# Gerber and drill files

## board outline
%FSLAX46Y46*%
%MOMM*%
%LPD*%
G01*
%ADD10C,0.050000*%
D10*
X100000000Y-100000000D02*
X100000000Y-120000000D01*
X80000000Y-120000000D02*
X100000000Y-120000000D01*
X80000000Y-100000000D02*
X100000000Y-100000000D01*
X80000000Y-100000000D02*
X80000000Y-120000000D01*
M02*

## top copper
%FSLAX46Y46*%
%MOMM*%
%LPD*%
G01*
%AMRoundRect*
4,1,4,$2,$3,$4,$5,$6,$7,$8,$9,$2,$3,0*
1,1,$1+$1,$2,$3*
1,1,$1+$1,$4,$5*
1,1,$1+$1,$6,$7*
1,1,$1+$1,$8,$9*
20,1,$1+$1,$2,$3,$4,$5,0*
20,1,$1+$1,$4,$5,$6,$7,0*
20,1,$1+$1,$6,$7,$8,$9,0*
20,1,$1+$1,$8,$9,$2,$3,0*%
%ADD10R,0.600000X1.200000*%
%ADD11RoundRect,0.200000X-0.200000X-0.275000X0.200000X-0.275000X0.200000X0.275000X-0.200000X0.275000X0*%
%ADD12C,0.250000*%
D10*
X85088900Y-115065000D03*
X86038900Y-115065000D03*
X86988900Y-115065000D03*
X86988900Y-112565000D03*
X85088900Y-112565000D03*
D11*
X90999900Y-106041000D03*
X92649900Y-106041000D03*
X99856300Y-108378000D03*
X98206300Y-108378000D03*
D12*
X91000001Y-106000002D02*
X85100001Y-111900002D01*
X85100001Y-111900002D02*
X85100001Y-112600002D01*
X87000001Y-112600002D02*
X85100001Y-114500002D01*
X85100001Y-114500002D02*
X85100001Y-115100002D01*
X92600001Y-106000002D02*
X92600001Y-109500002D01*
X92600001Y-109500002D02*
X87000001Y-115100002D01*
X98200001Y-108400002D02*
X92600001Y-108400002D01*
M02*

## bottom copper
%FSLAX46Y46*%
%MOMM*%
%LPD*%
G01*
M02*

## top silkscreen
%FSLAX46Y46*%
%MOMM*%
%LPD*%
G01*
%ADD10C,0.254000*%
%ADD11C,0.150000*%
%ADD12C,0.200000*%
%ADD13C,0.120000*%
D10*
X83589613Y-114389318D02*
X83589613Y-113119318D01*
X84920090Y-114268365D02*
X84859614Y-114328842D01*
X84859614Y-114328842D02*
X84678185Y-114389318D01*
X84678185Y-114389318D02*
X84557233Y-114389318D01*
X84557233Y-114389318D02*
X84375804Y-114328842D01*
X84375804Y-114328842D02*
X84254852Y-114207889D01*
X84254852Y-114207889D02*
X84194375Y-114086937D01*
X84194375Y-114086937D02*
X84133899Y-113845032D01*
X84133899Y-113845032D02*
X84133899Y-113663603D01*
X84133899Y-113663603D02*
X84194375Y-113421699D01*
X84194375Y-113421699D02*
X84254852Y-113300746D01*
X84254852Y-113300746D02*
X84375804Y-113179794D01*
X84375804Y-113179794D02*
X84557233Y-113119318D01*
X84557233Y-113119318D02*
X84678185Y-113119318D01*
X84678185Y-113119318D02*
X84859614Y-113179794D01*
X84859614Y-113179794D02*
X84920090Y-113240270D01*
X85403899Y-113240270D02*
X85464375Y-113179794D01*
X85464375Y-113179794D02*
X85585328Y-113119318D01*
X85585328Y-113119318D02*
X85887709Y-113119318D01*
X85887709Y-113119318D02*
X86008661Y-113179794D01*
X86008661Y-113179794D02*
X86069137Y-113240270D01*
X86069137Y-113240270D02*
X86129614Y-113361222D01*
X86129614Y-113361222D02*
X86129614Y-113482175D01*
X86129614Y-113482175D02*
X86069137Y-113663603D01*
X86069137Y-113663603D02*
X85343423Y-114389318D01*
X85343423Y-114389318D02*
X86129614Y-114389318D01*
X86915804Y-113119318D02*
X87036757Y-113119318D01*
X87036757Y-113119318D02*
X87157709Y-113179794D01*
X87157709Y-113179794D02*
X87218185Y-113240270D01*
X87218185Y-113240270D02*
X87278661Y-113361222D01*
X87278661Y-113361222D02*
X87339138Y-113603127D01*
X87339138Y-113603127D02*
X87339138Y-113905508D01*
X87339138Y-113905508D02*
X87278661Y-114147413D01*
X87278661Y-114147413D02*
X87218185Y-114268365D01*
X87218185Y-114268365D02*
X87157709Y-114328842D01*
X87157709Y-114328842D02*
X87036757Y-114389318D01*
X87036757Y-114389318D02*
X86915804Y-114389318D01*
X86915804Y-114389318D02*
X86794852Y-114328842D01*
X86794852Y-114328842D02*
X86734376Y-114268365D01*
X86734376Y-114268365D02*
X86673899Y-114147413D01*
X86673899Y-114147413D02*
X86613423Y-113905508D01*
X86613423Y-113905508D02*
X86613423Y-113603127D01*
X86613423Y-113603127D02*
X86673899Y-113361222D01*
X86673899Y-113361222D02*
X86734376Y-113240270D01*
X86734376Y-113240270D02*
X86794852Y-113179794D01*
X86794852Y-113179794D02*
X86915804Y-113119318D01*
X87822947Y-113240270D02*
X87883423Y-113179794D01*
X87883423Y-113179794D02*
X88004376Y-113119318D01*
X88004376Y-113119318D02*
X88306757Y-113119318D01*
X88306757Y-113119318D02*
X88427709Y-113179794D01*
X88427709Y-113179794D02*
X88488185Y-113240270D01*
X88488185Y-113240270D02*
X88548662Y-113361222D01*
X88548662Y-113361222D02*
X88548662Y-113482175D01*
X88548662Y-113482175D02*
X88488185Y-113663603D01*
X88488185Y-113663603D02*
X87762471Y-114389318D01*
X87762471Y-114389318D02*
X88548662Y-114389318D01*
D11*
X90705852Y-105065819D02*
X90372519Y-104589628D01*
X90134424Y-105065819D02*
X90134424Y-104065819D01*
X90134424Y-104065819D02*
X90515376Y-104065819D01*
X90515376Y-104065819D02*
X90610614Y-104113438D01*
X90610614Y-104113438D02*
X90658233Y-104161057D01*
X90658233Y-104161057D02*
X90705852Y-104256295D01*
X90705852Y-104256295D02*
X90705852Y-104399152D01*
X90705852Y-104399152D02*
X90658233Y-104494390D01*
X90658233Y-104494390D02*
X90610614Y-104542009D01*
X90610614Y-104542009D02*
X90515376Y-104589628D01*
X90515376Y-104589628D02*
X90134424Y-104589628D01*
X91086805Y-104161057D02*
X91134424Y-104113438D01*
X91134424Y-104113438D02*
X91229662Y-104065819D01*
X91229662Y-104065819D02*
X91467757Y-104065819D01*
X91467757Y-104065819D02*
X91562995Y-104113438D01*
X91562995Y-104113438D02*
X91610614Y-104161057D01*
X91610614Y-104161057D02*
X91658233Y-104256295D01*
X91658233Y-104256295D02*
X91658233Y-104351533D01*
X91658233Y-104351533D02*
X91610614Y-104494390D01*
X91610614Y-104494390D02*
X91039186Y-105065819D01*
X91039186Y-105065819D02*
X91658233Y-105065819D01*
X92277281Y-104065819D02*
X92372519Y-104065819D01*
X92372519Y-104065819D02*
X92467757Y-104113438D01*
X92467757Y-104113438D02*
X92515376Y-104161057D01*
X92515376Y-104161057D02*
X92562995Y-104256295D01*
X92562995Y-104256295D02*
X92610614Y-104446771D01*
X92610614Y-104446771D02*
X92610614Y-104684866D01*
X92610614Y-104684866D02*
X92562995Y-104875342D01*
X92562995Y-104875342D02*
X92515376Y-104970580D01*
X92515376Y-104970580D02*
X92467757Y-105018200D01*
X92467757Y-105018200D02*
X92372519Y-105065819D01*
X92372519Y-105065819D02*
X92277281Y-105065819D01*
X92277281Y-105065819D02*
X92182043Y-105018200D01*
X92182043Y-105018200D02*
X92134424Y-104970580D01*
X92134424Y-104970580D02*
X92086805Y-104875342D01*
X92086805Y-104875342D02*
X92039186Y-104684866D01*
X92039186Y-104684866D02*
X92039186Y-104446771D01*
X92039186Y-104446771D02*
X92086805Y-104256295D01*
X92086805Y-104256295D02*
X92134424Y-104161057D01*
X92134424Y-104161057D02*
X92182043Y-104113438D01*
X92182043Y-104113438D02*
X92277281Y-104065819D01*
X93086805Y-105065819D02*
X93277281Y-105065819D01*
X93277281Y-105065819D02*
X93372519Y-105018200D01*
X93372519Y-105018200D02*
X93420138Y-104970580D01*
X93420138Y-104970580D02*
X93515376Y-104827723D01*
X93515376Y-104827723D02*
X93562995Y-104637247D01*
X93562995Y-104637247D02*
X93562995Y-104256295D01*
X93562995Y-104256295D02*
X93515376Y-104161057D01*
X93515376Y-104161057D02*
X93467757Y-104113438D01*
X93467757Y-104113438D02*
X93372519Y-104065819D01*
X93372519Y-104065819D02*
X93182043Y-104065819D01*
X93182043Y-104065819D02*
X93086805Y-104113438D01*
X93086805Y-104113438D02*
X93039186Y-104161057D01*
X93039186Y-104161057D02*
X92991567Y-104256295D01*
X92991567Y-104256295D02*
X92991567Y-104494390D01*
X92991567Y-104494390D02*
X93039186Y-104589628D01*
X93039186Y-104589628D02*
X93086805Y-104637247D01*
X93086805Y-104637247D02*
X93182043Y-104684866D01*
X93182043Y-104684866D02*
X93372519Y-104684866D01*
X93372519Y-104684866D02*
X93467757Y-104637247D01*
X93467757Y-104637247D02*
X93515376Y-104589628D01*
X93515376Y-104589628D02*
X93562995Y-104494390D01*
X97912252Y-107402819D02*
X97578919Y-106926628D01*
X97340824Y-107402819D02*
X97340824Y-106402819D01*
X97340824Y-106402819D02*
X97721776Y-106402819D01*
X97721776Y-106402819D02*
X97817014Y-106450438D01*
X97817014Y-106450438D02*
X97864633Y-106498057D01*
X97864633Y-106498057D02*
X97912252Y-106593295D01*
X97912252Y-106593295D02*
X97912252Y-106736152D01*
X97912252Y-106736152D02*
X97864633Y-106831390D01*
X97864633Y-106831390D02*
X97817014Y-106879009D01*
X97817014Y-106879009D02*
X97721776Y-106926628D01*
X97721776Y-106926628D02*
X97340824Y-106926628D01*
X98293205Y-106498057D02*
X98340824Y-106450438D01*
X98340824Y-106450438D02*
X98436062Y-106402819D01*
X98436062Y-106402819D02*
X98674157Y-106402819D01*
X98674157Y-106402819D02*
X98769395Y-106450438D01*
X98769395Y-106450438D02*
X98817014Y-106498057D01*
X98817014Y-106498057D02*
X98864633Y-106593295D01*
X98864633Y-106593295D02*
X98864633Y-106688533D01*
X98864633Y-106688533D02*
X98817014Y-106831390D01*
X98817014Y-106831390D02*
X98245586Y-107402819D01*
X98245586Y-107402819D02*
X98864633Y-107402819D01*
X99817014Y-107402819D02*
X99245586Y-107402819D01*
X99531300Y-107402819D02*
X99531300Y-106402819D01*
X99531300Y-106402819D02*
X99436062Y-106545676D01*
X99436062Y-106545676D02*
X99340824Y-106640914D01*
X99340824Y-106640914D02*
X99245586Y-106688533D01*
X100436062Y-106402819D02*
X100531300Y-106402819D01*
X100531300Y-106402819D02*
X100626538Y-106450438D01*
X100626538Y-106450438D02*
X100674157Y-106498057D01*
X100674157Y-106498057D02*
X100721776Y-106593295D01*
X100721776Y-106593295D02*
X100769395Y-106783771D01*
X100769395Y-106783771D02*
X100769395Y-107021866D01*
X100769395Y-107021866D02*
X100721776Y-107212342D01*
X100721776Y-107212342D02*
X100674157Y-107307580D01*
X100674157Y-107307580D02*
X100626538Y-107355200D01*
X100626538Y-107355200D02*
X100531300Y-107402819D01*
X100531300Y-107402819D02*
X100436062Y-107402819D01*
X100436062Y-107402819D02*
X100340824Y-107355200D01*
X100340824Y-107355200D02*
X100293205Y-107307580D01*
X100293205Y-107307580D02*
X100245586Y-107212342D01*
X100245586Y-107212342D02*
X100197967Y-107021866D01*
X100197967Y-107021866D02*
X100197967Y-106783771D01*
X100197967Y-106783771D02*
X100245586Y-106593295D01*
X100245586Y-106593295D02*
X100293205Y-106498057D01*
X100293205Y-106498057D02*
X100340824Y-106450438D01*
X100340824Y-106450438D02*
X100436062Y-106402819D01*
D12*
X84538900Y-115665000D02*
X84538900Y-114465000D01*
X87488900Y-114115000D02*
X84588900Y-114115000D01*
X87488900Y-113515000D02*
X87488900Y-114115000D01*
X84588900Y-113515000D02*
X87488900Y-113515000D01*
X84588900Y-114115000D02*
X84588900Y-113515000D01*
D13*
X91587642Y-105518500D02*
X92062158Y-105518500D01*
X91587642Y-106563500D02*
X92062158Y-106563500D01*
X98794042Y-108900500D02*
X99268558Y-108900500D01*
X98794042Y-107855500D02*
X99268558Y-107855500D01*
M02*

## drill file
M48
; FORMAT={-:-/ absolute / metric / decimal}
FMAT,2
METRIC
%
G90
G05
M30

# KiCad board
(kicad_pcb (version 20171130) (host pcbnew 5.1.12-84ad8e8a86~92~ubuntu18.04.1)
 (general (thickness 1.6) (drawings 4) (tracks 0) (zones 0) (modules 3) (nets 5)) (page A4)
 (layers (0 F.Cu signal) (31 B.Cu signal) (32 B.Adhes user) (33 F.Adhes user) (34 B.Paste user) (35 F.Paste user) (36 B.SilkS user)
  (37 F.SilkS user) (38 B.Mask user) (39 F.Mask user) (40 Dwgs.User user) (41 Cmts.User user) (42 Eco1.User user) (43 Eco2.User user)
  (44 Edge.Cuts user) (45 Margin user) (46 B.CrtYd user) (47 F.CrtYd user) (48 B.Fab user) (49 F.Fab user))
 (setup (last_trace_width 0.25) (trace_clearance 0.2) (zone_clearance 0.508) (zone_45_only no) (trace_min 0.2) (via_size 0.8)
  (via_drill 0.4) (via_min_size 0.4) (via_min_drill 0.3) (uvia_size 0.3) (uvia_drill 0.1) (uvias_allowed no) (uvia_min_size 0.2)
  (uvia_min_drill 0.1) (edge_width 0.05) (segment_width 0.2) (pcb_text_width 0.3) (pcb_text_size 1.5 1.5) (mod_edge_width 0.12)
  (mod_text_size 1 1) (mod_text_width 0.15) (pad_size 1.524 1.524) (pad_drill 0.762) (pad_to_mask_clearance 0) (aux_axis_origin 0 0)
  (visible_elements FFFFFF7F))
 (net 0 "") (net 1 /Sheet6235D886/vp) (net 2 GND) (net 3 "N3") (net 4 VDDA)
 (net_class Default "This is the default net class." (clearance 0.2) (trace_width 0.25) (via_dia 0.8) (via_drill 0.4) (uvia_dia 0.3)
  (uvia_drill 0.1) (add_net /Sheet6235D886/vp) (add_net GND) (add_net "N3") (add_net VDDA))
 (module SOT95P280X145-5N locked (layer F.Cu) (at 86.038900 113.815000 90.000000)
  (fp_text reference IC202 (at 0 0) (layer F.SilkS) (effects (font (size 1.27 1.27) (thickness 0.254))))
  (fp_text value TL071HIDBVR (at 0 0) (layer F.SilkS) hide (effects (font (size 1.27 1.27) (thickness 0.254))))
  (fp_line (start -1.85 -1.5) (end -0.65 -1.5) (layer F.SilkS) (width 0.2))
  (fp_line (start -0.3 1.45) (end -0.3 -1.45) (layer F.SilkS) (width 0.2))
  (fp_line (start 0.3 1.45) (end -0.3 1.45) (layer F.SilkS) (width 0.2))
  (fp_line (start 0.3 -1.45) (end 0.3 1.45) (layer F.SilkS) (width 0.2))
  (fp_line (start -0.3 -1.45) (end 0.3 -1.45) (layer F.SilkS) (width 0.2))
  (pad 1 smd rect (at -1.25 -0.95 180.000000) (size 0.6 1.2) (layers F.Cu F.Mask F.Paste) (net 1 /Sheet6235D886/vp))
  (pad 2 smd rect (at -1.25 0 180.000000) (size 0.6 1.2) (layers F.Cu F.Mask F.Paste) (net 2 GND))
  (pad 3 smd rect (at -1.25 0.95 180.000000) (size 0.6 1.2) (layers F.Cu F.Mask F.Paste) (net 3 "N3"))
  (pad 4 smd rect (at 1.25 0.95 180.000000) (size 0.6 1.2) (layers F.Cu F.Mask F.Paste) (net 1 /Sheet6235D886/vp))
  (pad 5 smd rect (at 1.25 -0.95 180.000000) (size 0.6 1.2) (layers F.Cu F.Mask F.Paste) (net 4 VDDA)))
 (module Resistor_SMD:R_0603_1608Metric (layer F.Cu) (at 91.824900 106.041000)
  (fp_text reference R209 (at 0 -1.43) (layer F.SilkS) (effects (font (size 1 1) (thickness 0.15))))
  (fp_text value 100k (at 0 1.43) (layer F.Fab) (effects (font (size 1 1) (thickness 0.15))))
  (fp_line (start -0.237258 -0.5225) (end 0.237258 -0.5225) (layer F.SilkS) (width 0.12))
  (fp_line (start -0.237258 0.5225) (end 0.237258 0.5225) (layer F.SilkS) (width 0.12))
  (pad 1 smd roundrect (at -0.825 0) (size 0.8 0.95) (layers F.Cu F.Mask F.Paste) (roundrect_rratio 0.25) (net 4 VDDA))
  (pad 2 smd roundrect (at 0.825 0) (size 0.8 0.95) (layers F.Cu F.Mask F.Paste) (roundrect_rratio 0.25) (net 3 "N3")))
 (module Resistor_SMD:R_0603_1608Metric (layer F.Cu) (at 99.031300 108.378000)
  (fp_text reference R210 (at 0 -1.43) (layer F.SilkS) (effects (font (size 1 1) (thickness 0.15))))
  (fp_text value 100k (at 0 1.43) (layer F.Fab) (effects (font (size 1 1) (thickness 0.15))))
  (fp_line (start -0.237258 0.5225) (end 0.237258 0.5225) (layer F.SilkS) (width 0.12))
  (fp_line (start -0.237258 -0.5225) (end 0.237258 -0.5225) (layer F.SilkS) (width 0.12))
  (pad 2 smd roundrect (at 0.825 0) (size 0.8 0.95) (layers F.Cu F.Mask F.Paste) (roundrect_rratio 0.25) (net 2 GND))
  (pad 1 smd roundrect (at -0.825 0) (size 0.8 0.95) (layers F.Cu F.Mask F.Paste) (roundrect_rratio 0.25) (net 3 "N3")))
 (gr_line (start 100 100) (end 100 120) (layer Edge.Cuts) (width 0.05))
 (gr_line (start 80 120) (end 100 120) (layer Edge.Cuts) (width 0.05))
 (gr_line (start 80 100) (end 100 100) (layer Edge.Cuts) (width 0.05))
 (gr_line (start 80 100) (end 80 120) (layer Edge.Cuts) (width 0.05))
 (segment (start 91.000001 106.000002) (end 85.100001 111.900002) (width 0.250000) (layer F.Cu) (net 4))
 (segment (start 85.100001 111.900002) (end 85.100001 112.600002) (width 0.250000) (layer F.Cu) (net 4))
 (segment (start 87.000001 112.600002) (end 85.100001 114.500002) (width 0.250000) (layer F.Cu) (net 1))
 (segment (start 85.100001 114.500002) (end 85.100001 115.100002) (width 0.250000) (layer F.Cu) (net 1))
 (segment (start 92.600001 106.000002) (end 92.600001 109.500002) (width 0.250000) (layer F.Cu) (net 3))
 (segment (start 92.600001 109.500002) (end 87.000001 115.100002) (width 0.250000) (layer F.Cu) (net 3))
 (segment (start 98.200001 108.400002) (end 92.600001 108.400002) (width 0.250000) (layer F.Cu) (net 3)))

